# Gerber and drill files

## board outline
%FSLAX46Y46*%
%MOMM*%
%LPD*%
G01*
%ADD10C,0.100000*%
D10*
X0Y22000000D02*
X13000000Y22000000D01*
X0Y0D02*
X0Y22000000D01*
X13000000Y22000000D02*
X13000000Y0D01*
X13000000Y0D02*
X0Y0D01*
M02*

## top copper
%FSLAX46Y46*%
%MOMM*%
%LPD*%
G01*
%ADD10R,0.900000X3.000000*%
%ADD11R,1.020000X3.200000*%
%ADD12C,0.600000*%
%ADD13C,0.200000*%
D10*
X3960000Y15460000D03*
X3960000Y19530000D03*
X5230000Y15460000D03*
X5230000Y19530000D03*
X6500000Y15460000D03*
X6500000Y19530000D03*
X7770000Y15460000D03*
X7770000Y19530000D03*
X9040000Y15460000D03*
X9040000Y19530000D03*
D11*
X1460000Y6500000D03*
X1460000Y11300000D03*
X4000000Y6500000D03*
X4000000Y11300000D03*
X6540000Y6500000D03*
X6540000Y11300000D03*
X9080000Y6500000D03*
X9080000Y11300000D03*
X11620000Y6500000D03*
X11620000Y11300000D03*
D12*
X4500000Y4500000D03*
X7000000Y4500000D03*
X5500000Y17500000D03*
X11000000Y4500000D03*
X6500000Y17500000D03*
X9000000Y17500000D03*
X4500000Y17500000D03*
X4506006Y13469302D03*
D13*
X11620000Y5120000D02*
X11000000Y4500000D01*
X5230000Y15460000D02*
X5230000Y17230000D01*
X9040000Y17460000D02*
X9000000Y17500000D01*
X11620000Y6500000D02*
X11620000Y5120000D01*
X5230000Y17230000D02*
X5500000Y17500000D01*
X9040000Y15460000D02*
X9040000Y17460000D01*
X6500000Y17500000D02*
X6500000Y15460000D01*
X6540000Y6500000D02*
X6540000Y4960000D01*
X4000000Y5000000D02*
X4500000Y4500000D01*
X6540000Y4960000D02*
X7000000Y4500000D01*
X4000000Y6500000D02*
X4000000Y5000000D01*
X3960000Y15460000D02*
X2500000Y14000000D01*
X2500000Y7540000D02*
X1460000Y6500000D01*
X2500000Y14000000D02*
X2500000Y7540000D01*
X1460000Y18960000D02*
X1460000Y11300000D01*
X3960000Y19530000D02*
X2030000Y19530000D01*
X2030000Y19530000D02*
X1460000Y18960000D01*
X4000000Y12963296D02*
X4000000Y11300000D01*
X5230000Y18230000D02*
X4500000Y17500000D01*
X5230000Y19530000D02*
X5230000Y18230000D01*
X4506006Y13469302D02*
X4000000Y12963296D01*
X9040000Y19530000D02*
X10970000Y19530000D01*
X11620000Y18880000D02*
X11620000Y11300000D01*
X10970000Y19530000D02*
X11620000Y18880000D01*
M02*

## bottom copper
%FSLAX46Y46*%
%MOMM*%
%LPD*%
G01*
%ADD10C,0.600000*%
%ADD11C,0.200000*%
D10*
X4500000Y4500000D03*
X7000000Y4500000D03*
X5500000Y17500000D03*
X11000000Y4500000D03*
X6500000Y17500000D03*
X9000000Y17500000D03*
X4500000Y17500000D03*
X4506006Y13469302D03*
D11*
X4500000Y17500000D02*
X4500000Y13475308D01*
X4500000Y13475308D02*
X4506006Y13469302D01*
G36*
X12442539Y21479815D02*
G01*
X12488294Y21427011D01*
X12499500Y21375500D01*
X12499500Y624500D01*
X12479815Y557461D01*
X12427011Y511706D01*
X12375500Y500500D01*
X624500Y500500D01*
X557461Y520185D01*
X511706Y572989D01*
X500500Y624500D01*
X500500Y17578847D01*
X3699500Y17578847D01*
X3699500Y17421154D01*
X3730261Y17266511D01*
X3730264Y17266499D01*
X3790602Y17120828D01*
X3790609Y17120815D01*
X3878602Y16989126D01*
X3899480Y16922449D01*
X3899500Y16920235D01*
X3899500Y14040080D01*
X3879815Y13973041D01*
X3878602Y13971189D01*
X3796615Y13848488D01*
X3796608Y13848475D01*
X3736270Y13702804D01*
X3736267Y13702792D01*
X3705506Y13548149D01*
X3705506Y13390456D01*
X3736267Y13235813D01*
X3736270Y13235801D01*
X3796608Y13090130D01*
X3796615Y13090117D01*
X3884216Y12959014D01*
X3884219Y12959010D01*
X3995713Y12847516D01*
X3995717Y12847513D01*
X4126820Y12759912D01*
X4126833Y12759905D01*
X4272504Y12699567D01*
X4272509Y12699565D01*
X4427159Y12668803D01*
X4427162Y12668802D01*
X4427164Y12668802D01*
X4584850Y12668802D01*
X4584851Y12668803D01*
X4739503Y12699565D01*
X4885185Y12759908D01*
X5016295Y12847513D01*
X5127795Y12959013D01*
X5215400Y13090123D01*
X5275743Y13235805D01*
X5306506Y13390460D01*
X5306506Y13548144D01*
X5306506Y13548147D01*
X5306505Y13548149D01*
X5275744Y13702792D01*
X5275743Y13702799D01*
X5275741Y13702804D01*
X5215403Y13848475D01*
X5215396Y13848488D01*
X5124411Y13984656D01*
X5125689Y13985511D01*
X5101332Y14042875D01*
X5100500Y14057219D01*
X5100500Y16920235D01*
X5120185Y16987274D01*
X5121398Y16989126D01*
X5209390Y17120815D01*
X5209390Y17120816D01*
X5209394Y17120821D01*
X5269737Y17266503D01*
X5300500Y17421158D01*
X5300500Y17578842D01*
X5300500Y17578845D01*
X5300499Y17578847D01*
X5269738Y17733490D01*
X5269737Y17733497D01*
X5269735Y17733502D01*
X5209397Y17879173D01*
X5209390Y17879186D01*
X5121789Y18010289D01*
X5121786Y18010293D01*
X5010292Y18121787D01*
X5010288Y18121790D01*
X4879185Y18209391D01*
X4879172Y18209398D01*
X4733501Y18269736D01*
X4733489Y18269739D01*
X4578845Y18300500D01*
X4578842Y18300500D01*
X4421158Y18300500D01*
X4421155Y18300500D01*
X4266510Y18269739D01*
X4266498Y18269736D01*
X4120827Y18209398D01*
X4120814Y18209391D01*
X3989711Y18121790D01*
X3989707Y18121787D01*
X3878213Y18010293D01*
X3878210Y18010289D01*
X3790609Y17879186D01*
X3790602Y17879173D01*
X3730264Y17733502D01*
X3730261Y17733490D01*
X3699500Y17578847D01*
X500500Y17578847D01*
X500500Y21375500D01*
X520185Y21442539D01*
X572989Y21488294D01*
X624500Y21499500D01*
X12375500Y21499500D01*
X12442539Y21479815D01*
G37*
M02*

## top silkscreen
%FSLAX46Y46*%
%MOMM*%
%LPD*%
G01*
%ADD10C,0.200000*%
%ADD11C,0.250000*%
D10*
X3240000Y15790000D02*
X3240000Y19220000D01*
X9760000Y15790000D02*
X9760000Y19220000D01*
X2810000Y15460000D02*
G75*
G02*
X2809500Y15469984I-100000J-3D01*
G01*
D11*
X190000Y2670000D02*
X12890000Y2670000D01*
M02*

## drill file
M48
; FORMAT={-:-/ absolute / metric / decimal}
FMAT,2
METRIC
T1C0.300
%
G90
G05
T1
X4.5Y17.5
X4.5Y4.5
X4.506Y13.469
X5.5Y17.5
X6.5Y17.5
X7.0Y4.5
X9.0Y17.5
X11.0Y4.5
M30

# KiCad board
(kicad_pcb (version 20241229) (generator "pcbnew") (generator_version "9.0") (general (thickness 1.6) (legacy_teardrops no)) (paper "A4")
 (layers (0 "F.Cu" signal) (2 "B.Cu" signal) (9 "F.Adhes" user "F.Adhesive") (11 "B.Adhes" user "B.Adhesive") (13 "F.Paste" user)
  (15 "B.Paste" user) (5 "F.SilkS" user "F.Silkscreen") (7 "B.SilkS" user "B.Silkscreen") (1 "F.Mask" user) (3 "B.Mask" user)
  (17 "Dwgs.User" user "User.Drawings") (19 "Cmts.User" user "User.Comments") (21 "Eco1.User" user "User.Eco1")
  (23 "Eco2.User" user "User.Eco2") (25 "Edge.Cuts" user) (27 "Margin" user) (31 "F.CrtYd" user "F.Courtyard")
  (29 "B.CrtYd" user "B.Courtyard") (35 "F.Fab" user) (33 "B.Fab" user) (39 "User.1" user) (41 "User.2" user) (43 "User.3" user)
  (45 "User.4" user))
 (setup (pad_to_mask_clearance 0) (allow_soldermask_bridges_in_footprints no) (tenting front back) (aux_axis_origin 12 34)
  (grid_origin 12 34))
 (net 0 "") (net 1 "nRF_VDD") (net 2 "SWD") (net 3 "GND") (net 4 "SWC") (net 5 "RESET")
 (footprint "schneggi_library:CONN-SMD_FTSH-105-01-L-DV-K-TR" (layer "F.Cu") (at 18.5 16.5)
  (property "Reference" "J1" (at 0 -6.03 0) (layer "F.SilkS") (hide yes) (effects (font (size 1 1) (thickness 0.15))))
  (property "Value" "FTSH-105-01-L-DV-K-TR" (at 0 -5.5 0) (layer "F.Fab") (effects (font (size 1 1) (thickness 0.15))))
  (fp_line (start -3.26 1.71) (end -3.26 -1.72) (stroke (width 0.2) (type solid)) (layer "F.SilkS"))
  (fp_line (start 3.26 1.71) (end 3.26 -1.72) (stroke (width 0.2) (type solid)) (layer "F.SilkS"))
  (fp_arc (start -3.69 2.04) (mid -3.889875 2.044998) (end -3.6905 2.030016) (stroke (width 0.2) (type solid)) (layer "F.SilkS"))
  (pad "1" smd rect (at -2.54 2.04) (size 0.9 3) (layers "F.Cu" "F.Mask" "F.Paste") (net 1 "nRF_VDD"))
  (pad "2" smd rect (at -2.54 -2.03) (size 0.9 3) (layers "F.Cu" "F.Mask" "F.Paste") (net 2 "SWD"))
  (pad "3" smd rect (at -1.27 2.04) (size 0.9 3) (layers "F.Cu" "F.Mask" "F.Paste") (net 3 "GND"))
  (pad "4" smd rect (at -1.27 -2.03) (size 0.9 3) (layers "F.Cu" "F.Mask" "F.Paste") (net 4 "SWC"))
  (pad "5" smd rect (at 0 2.04) (size 0.9 3) (layers "F.Cu" "F.Mask" "F.Paste") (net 3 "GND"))
  (pad "6" smd rect (at 0 -2.03) (size 0.9 3) (layers "F.Cu" "F.Mask" "F.Paste"))
  (pad "7" smd rect (at 1.27 2.04) (size 0.9 3) (layers "F.Cu" "F.Mask" "F.Paste"))
  (pad "8" smd rect (at 1.27 -2.03) (size 0.9 3) (layers "F.Cu" "F.Mask" "F.Paste"))
  (pad "9" smd rect (at 2.54 2.04) (size 0.9 3) (layers "F.Cu" "F.Mask" "F.Paste") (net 3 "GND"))
  (pad "10" smd rect (at 2.54 -2.03) (size 0.9 3) (layers "F.Cu" "F.Mask" "F.Paste") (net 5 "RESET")))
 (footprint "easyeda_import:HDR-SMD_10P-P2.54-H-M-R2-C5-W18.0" (layer "F.Cu") (at 18.54 25.1)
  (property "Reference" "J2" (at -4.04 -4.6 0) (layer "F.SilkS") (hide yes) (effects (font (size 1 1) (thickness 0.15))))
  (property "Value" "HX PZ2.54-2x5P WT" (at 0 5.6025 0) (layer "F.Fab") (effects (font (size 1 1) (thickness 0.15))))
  (fp_line (start -6.35 6.23) (end 6.35 6.23) (stroke (width 0.25) (type solid)) (layer "F.SilkS"))
  (pad "1" smd rect (at -5.08 2.4) (size 1.02 3.2) (layers "F.Cu" "F.Mask" "F.Paste") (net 1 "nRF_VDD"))
  (pad "2" smd rect (at -5.08 -2.4) (size 1.02 3.2) (layers "F.Cu" "F.Mask" "F.Paste") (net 2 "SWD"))
  (pad "3" smd rect (at -2.54 2.4) (size 1.02 3.2) (layers "F.Cu" "F.Mask" "F.Paste") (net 3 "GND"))
  (pad "4" smd rect (at -2.54 -2.4) (size 1.02 3.2) (layers "F.Cu" "F.Mask" "F.Paste") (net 4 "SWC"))
  (pad "5" smd rect (at 0 2.4) (size 1.02 3.2) (layers "F.Cu" "F.Mask" "F.Paste") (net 3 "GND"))
  (pad "6" smd rect (at 0 -2.4) (size 1.02 3.2) (layers "F.Cu" "F.Mask" "F.Paste"))
  (pad "7" smd rect (at 2.54 2.4) (size 1.02 3.2) (layers "F.Cu" "F.Mask" "F.Paste"))
  (pad "8" smd rect (at 2.54 -2.4) (size 1.02 3.2) (layers "F.Cu" "F.Mask" "F.Paste"))
  (pad "9" smd rect (at 5.08 2.4) (size 1.02 3.2) (layers "F.Cu" "F.Mask" "F.Paste") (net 3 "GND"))
  (pad "10" smd rect (at 5.08 -2.4) (size 1.02 3.2) (layers "F.Cu" "F.Mask" "F.Paste") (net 5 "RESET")))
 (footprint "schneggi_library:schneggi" (layer "B.Cu") (at 18.5 29.5 180)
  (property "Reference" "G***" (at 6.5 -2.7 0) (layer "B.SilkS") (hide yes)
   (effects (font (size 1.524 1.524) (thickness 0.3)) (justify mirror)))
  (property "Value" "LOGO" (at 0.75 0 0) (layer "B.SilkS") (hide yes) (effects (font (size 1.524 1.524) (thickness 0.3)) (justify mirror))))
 (gr_line (start 12 12) (end 25 12) (stroke (width 0.1) (type default)) (layer "Edge.Cuts"))
 (gr_line (start 12 34) (end 12 12) (stroke (width 0.1) (type default)) (layer "Edge.Cuts"))
 (gr_line (start 25 12) (end 25 34) (stroke (width 0.1) (type default)) (layer "Edge.Cuts"))
 (gr_line (start 25 34) (end 12 34) (stroke (width 0.1) (type default)) (layer "Edge.Cuts"))
 (segment (start 23.62 28.88) (end 23 29.5) (width 0.2) (layer "F.Cu") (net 3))
 (segment (start 17.23 18.54) (end 17.23 16.77) (width 0.2) (layer "F.Cu") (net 3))
 (segment (start 21.04 16.54) (end 21 16.5) (width 0.2) (layer "F.Cu") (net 3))
 (segment (start 23.62 27.5) (end 23.62 28.88) (width 0.2) (layer "F.Cu") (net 3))
 (segment (start 17.23 16.77) (end 17.5 16.5) (width 0.2) (layer "F.Cu") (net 3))
 (segment (start 21.04 18.54) (end 21.04 16.54) (width 0.2) (layer "F.Cu") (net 3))
 (segment (start 18.5 16.5) (end 18.5 18.54) (width 0.2) (layer "F.Cu") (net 3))
 (segment (start 18.54 27.5) (end 18.54 29.04) (width 0.2) (layer "F.Cu") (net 3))
 (segment (start 16 29) (end 16.5 29.5) (width 0.2) (layer "F.Cu") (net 3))
 (segment (start 18.54 29.04) (end 19 29.5) (width 0.2) (layer "F.Cu") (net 3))
 (segment (start 16 27.5) (end 16 29) (width 0.2) (layer "F.Cu") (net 3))
 (via (at 16.5 29.5) (size 0.6) (drill 0.3) (layers "F.Cu" "B.Cu") (free yes) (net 3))
 (via (at 19 29.5) (size 0.6) (drill 0.3) (layers "F.Cu" "B.Cu") (free yes) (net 3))
 (via (at 17.5 16.5) (size 0.6) (drill 0.3) (layers "F.Cu" "B.Cu") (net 3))
 (via (at 23 29.5) (size 0.6) (drill 0.3) (layers "F.Cu" "B.Cu") (free yes) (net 3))
 (via (at 18.5 16.5) (size 0.6) (drill 0.3) (layers "F.Cu" "B.Cu") (free yes) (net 3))
 (via (at 21 16.5) (size 0.6) (drill 0.3) (layers "F.Cu" "B.Cu") (free yes) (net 3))
 (segment (start 15.96 18.54) (end 14.5 20) (width 0.2) (layer "F.Cu") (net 1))
 (segment (start 14.5 26.46) (end 13.46 27.5) (width 0.2) (layer "F.Cu") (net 1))
 (segment (start 14.5 20) (end 14.5 26.46) (width 0.2) (layer "F.Cu") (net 1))
 (segment (start 13.46 15.04) (end 13.46 22.7) (width 0.2) (layer "F.Cu") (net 2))
 (segment (start 15.96 14.47) (end 14.03 14.47) (width 0.2) (layer "F.Cu") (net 2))
 (segment (start 14.03 14.47) (end 13.46 15.04) (width 0.2) (layer "F.Cu") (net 2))
 (segment (start 16 21.036704) (end 16 22.7) (width 0.2) (layer "F.Cu") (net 4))
 (segment (start 17.23 15.77) (end 16.5 16.5) (width 0.2) (layer "F.Cu") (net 4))
 (segment (start 17.23 14.47) (end 17.23 15.77) (width 0.2) (layer "F.Cu") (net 4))
 (segment (start 16.506006 20.530698) (end 16 21.036704) (width 0.2) (layer "F.Cu") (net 4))
 (via (at 16.5 16.5) (size 0.6) (drill 0.3) (layers "F.Cu" "B.Cu") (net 4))
 (via (at 16.506006 20.530698) (size 0.6) (drill 0.3) (layers "F.Cu" "B.Cu") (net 4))
 (segment (start 16.5 16.5) (end 16.5 20.524692) (width 0.2) (layer "B.Cu") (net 4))
 (segment (start 16.5 20.524692) (end 16.506006 20.530698) (width 0.2) (layer "B.Cu") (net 4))
 (segment (start 21.04 14.47) (end 22.97 14.47) (width 0.2) (layer "F.Cu") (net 5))
 (segment (start 23.62 15.12) (end 23.62 22.7) (width 0.2) (layer "F.Cu") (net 5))
 (segment (start 22.97 14.47) (end 23.62 15.12) (width 0.2) (layer "F.Cu") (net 5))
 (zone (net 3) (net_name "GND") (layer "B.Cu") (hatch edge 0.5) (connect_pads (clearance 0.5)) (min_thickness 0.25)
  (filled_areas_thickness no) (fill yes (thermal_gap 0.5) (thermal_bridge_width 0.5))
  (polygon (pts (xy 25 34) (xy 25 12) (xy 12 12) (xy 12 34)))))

